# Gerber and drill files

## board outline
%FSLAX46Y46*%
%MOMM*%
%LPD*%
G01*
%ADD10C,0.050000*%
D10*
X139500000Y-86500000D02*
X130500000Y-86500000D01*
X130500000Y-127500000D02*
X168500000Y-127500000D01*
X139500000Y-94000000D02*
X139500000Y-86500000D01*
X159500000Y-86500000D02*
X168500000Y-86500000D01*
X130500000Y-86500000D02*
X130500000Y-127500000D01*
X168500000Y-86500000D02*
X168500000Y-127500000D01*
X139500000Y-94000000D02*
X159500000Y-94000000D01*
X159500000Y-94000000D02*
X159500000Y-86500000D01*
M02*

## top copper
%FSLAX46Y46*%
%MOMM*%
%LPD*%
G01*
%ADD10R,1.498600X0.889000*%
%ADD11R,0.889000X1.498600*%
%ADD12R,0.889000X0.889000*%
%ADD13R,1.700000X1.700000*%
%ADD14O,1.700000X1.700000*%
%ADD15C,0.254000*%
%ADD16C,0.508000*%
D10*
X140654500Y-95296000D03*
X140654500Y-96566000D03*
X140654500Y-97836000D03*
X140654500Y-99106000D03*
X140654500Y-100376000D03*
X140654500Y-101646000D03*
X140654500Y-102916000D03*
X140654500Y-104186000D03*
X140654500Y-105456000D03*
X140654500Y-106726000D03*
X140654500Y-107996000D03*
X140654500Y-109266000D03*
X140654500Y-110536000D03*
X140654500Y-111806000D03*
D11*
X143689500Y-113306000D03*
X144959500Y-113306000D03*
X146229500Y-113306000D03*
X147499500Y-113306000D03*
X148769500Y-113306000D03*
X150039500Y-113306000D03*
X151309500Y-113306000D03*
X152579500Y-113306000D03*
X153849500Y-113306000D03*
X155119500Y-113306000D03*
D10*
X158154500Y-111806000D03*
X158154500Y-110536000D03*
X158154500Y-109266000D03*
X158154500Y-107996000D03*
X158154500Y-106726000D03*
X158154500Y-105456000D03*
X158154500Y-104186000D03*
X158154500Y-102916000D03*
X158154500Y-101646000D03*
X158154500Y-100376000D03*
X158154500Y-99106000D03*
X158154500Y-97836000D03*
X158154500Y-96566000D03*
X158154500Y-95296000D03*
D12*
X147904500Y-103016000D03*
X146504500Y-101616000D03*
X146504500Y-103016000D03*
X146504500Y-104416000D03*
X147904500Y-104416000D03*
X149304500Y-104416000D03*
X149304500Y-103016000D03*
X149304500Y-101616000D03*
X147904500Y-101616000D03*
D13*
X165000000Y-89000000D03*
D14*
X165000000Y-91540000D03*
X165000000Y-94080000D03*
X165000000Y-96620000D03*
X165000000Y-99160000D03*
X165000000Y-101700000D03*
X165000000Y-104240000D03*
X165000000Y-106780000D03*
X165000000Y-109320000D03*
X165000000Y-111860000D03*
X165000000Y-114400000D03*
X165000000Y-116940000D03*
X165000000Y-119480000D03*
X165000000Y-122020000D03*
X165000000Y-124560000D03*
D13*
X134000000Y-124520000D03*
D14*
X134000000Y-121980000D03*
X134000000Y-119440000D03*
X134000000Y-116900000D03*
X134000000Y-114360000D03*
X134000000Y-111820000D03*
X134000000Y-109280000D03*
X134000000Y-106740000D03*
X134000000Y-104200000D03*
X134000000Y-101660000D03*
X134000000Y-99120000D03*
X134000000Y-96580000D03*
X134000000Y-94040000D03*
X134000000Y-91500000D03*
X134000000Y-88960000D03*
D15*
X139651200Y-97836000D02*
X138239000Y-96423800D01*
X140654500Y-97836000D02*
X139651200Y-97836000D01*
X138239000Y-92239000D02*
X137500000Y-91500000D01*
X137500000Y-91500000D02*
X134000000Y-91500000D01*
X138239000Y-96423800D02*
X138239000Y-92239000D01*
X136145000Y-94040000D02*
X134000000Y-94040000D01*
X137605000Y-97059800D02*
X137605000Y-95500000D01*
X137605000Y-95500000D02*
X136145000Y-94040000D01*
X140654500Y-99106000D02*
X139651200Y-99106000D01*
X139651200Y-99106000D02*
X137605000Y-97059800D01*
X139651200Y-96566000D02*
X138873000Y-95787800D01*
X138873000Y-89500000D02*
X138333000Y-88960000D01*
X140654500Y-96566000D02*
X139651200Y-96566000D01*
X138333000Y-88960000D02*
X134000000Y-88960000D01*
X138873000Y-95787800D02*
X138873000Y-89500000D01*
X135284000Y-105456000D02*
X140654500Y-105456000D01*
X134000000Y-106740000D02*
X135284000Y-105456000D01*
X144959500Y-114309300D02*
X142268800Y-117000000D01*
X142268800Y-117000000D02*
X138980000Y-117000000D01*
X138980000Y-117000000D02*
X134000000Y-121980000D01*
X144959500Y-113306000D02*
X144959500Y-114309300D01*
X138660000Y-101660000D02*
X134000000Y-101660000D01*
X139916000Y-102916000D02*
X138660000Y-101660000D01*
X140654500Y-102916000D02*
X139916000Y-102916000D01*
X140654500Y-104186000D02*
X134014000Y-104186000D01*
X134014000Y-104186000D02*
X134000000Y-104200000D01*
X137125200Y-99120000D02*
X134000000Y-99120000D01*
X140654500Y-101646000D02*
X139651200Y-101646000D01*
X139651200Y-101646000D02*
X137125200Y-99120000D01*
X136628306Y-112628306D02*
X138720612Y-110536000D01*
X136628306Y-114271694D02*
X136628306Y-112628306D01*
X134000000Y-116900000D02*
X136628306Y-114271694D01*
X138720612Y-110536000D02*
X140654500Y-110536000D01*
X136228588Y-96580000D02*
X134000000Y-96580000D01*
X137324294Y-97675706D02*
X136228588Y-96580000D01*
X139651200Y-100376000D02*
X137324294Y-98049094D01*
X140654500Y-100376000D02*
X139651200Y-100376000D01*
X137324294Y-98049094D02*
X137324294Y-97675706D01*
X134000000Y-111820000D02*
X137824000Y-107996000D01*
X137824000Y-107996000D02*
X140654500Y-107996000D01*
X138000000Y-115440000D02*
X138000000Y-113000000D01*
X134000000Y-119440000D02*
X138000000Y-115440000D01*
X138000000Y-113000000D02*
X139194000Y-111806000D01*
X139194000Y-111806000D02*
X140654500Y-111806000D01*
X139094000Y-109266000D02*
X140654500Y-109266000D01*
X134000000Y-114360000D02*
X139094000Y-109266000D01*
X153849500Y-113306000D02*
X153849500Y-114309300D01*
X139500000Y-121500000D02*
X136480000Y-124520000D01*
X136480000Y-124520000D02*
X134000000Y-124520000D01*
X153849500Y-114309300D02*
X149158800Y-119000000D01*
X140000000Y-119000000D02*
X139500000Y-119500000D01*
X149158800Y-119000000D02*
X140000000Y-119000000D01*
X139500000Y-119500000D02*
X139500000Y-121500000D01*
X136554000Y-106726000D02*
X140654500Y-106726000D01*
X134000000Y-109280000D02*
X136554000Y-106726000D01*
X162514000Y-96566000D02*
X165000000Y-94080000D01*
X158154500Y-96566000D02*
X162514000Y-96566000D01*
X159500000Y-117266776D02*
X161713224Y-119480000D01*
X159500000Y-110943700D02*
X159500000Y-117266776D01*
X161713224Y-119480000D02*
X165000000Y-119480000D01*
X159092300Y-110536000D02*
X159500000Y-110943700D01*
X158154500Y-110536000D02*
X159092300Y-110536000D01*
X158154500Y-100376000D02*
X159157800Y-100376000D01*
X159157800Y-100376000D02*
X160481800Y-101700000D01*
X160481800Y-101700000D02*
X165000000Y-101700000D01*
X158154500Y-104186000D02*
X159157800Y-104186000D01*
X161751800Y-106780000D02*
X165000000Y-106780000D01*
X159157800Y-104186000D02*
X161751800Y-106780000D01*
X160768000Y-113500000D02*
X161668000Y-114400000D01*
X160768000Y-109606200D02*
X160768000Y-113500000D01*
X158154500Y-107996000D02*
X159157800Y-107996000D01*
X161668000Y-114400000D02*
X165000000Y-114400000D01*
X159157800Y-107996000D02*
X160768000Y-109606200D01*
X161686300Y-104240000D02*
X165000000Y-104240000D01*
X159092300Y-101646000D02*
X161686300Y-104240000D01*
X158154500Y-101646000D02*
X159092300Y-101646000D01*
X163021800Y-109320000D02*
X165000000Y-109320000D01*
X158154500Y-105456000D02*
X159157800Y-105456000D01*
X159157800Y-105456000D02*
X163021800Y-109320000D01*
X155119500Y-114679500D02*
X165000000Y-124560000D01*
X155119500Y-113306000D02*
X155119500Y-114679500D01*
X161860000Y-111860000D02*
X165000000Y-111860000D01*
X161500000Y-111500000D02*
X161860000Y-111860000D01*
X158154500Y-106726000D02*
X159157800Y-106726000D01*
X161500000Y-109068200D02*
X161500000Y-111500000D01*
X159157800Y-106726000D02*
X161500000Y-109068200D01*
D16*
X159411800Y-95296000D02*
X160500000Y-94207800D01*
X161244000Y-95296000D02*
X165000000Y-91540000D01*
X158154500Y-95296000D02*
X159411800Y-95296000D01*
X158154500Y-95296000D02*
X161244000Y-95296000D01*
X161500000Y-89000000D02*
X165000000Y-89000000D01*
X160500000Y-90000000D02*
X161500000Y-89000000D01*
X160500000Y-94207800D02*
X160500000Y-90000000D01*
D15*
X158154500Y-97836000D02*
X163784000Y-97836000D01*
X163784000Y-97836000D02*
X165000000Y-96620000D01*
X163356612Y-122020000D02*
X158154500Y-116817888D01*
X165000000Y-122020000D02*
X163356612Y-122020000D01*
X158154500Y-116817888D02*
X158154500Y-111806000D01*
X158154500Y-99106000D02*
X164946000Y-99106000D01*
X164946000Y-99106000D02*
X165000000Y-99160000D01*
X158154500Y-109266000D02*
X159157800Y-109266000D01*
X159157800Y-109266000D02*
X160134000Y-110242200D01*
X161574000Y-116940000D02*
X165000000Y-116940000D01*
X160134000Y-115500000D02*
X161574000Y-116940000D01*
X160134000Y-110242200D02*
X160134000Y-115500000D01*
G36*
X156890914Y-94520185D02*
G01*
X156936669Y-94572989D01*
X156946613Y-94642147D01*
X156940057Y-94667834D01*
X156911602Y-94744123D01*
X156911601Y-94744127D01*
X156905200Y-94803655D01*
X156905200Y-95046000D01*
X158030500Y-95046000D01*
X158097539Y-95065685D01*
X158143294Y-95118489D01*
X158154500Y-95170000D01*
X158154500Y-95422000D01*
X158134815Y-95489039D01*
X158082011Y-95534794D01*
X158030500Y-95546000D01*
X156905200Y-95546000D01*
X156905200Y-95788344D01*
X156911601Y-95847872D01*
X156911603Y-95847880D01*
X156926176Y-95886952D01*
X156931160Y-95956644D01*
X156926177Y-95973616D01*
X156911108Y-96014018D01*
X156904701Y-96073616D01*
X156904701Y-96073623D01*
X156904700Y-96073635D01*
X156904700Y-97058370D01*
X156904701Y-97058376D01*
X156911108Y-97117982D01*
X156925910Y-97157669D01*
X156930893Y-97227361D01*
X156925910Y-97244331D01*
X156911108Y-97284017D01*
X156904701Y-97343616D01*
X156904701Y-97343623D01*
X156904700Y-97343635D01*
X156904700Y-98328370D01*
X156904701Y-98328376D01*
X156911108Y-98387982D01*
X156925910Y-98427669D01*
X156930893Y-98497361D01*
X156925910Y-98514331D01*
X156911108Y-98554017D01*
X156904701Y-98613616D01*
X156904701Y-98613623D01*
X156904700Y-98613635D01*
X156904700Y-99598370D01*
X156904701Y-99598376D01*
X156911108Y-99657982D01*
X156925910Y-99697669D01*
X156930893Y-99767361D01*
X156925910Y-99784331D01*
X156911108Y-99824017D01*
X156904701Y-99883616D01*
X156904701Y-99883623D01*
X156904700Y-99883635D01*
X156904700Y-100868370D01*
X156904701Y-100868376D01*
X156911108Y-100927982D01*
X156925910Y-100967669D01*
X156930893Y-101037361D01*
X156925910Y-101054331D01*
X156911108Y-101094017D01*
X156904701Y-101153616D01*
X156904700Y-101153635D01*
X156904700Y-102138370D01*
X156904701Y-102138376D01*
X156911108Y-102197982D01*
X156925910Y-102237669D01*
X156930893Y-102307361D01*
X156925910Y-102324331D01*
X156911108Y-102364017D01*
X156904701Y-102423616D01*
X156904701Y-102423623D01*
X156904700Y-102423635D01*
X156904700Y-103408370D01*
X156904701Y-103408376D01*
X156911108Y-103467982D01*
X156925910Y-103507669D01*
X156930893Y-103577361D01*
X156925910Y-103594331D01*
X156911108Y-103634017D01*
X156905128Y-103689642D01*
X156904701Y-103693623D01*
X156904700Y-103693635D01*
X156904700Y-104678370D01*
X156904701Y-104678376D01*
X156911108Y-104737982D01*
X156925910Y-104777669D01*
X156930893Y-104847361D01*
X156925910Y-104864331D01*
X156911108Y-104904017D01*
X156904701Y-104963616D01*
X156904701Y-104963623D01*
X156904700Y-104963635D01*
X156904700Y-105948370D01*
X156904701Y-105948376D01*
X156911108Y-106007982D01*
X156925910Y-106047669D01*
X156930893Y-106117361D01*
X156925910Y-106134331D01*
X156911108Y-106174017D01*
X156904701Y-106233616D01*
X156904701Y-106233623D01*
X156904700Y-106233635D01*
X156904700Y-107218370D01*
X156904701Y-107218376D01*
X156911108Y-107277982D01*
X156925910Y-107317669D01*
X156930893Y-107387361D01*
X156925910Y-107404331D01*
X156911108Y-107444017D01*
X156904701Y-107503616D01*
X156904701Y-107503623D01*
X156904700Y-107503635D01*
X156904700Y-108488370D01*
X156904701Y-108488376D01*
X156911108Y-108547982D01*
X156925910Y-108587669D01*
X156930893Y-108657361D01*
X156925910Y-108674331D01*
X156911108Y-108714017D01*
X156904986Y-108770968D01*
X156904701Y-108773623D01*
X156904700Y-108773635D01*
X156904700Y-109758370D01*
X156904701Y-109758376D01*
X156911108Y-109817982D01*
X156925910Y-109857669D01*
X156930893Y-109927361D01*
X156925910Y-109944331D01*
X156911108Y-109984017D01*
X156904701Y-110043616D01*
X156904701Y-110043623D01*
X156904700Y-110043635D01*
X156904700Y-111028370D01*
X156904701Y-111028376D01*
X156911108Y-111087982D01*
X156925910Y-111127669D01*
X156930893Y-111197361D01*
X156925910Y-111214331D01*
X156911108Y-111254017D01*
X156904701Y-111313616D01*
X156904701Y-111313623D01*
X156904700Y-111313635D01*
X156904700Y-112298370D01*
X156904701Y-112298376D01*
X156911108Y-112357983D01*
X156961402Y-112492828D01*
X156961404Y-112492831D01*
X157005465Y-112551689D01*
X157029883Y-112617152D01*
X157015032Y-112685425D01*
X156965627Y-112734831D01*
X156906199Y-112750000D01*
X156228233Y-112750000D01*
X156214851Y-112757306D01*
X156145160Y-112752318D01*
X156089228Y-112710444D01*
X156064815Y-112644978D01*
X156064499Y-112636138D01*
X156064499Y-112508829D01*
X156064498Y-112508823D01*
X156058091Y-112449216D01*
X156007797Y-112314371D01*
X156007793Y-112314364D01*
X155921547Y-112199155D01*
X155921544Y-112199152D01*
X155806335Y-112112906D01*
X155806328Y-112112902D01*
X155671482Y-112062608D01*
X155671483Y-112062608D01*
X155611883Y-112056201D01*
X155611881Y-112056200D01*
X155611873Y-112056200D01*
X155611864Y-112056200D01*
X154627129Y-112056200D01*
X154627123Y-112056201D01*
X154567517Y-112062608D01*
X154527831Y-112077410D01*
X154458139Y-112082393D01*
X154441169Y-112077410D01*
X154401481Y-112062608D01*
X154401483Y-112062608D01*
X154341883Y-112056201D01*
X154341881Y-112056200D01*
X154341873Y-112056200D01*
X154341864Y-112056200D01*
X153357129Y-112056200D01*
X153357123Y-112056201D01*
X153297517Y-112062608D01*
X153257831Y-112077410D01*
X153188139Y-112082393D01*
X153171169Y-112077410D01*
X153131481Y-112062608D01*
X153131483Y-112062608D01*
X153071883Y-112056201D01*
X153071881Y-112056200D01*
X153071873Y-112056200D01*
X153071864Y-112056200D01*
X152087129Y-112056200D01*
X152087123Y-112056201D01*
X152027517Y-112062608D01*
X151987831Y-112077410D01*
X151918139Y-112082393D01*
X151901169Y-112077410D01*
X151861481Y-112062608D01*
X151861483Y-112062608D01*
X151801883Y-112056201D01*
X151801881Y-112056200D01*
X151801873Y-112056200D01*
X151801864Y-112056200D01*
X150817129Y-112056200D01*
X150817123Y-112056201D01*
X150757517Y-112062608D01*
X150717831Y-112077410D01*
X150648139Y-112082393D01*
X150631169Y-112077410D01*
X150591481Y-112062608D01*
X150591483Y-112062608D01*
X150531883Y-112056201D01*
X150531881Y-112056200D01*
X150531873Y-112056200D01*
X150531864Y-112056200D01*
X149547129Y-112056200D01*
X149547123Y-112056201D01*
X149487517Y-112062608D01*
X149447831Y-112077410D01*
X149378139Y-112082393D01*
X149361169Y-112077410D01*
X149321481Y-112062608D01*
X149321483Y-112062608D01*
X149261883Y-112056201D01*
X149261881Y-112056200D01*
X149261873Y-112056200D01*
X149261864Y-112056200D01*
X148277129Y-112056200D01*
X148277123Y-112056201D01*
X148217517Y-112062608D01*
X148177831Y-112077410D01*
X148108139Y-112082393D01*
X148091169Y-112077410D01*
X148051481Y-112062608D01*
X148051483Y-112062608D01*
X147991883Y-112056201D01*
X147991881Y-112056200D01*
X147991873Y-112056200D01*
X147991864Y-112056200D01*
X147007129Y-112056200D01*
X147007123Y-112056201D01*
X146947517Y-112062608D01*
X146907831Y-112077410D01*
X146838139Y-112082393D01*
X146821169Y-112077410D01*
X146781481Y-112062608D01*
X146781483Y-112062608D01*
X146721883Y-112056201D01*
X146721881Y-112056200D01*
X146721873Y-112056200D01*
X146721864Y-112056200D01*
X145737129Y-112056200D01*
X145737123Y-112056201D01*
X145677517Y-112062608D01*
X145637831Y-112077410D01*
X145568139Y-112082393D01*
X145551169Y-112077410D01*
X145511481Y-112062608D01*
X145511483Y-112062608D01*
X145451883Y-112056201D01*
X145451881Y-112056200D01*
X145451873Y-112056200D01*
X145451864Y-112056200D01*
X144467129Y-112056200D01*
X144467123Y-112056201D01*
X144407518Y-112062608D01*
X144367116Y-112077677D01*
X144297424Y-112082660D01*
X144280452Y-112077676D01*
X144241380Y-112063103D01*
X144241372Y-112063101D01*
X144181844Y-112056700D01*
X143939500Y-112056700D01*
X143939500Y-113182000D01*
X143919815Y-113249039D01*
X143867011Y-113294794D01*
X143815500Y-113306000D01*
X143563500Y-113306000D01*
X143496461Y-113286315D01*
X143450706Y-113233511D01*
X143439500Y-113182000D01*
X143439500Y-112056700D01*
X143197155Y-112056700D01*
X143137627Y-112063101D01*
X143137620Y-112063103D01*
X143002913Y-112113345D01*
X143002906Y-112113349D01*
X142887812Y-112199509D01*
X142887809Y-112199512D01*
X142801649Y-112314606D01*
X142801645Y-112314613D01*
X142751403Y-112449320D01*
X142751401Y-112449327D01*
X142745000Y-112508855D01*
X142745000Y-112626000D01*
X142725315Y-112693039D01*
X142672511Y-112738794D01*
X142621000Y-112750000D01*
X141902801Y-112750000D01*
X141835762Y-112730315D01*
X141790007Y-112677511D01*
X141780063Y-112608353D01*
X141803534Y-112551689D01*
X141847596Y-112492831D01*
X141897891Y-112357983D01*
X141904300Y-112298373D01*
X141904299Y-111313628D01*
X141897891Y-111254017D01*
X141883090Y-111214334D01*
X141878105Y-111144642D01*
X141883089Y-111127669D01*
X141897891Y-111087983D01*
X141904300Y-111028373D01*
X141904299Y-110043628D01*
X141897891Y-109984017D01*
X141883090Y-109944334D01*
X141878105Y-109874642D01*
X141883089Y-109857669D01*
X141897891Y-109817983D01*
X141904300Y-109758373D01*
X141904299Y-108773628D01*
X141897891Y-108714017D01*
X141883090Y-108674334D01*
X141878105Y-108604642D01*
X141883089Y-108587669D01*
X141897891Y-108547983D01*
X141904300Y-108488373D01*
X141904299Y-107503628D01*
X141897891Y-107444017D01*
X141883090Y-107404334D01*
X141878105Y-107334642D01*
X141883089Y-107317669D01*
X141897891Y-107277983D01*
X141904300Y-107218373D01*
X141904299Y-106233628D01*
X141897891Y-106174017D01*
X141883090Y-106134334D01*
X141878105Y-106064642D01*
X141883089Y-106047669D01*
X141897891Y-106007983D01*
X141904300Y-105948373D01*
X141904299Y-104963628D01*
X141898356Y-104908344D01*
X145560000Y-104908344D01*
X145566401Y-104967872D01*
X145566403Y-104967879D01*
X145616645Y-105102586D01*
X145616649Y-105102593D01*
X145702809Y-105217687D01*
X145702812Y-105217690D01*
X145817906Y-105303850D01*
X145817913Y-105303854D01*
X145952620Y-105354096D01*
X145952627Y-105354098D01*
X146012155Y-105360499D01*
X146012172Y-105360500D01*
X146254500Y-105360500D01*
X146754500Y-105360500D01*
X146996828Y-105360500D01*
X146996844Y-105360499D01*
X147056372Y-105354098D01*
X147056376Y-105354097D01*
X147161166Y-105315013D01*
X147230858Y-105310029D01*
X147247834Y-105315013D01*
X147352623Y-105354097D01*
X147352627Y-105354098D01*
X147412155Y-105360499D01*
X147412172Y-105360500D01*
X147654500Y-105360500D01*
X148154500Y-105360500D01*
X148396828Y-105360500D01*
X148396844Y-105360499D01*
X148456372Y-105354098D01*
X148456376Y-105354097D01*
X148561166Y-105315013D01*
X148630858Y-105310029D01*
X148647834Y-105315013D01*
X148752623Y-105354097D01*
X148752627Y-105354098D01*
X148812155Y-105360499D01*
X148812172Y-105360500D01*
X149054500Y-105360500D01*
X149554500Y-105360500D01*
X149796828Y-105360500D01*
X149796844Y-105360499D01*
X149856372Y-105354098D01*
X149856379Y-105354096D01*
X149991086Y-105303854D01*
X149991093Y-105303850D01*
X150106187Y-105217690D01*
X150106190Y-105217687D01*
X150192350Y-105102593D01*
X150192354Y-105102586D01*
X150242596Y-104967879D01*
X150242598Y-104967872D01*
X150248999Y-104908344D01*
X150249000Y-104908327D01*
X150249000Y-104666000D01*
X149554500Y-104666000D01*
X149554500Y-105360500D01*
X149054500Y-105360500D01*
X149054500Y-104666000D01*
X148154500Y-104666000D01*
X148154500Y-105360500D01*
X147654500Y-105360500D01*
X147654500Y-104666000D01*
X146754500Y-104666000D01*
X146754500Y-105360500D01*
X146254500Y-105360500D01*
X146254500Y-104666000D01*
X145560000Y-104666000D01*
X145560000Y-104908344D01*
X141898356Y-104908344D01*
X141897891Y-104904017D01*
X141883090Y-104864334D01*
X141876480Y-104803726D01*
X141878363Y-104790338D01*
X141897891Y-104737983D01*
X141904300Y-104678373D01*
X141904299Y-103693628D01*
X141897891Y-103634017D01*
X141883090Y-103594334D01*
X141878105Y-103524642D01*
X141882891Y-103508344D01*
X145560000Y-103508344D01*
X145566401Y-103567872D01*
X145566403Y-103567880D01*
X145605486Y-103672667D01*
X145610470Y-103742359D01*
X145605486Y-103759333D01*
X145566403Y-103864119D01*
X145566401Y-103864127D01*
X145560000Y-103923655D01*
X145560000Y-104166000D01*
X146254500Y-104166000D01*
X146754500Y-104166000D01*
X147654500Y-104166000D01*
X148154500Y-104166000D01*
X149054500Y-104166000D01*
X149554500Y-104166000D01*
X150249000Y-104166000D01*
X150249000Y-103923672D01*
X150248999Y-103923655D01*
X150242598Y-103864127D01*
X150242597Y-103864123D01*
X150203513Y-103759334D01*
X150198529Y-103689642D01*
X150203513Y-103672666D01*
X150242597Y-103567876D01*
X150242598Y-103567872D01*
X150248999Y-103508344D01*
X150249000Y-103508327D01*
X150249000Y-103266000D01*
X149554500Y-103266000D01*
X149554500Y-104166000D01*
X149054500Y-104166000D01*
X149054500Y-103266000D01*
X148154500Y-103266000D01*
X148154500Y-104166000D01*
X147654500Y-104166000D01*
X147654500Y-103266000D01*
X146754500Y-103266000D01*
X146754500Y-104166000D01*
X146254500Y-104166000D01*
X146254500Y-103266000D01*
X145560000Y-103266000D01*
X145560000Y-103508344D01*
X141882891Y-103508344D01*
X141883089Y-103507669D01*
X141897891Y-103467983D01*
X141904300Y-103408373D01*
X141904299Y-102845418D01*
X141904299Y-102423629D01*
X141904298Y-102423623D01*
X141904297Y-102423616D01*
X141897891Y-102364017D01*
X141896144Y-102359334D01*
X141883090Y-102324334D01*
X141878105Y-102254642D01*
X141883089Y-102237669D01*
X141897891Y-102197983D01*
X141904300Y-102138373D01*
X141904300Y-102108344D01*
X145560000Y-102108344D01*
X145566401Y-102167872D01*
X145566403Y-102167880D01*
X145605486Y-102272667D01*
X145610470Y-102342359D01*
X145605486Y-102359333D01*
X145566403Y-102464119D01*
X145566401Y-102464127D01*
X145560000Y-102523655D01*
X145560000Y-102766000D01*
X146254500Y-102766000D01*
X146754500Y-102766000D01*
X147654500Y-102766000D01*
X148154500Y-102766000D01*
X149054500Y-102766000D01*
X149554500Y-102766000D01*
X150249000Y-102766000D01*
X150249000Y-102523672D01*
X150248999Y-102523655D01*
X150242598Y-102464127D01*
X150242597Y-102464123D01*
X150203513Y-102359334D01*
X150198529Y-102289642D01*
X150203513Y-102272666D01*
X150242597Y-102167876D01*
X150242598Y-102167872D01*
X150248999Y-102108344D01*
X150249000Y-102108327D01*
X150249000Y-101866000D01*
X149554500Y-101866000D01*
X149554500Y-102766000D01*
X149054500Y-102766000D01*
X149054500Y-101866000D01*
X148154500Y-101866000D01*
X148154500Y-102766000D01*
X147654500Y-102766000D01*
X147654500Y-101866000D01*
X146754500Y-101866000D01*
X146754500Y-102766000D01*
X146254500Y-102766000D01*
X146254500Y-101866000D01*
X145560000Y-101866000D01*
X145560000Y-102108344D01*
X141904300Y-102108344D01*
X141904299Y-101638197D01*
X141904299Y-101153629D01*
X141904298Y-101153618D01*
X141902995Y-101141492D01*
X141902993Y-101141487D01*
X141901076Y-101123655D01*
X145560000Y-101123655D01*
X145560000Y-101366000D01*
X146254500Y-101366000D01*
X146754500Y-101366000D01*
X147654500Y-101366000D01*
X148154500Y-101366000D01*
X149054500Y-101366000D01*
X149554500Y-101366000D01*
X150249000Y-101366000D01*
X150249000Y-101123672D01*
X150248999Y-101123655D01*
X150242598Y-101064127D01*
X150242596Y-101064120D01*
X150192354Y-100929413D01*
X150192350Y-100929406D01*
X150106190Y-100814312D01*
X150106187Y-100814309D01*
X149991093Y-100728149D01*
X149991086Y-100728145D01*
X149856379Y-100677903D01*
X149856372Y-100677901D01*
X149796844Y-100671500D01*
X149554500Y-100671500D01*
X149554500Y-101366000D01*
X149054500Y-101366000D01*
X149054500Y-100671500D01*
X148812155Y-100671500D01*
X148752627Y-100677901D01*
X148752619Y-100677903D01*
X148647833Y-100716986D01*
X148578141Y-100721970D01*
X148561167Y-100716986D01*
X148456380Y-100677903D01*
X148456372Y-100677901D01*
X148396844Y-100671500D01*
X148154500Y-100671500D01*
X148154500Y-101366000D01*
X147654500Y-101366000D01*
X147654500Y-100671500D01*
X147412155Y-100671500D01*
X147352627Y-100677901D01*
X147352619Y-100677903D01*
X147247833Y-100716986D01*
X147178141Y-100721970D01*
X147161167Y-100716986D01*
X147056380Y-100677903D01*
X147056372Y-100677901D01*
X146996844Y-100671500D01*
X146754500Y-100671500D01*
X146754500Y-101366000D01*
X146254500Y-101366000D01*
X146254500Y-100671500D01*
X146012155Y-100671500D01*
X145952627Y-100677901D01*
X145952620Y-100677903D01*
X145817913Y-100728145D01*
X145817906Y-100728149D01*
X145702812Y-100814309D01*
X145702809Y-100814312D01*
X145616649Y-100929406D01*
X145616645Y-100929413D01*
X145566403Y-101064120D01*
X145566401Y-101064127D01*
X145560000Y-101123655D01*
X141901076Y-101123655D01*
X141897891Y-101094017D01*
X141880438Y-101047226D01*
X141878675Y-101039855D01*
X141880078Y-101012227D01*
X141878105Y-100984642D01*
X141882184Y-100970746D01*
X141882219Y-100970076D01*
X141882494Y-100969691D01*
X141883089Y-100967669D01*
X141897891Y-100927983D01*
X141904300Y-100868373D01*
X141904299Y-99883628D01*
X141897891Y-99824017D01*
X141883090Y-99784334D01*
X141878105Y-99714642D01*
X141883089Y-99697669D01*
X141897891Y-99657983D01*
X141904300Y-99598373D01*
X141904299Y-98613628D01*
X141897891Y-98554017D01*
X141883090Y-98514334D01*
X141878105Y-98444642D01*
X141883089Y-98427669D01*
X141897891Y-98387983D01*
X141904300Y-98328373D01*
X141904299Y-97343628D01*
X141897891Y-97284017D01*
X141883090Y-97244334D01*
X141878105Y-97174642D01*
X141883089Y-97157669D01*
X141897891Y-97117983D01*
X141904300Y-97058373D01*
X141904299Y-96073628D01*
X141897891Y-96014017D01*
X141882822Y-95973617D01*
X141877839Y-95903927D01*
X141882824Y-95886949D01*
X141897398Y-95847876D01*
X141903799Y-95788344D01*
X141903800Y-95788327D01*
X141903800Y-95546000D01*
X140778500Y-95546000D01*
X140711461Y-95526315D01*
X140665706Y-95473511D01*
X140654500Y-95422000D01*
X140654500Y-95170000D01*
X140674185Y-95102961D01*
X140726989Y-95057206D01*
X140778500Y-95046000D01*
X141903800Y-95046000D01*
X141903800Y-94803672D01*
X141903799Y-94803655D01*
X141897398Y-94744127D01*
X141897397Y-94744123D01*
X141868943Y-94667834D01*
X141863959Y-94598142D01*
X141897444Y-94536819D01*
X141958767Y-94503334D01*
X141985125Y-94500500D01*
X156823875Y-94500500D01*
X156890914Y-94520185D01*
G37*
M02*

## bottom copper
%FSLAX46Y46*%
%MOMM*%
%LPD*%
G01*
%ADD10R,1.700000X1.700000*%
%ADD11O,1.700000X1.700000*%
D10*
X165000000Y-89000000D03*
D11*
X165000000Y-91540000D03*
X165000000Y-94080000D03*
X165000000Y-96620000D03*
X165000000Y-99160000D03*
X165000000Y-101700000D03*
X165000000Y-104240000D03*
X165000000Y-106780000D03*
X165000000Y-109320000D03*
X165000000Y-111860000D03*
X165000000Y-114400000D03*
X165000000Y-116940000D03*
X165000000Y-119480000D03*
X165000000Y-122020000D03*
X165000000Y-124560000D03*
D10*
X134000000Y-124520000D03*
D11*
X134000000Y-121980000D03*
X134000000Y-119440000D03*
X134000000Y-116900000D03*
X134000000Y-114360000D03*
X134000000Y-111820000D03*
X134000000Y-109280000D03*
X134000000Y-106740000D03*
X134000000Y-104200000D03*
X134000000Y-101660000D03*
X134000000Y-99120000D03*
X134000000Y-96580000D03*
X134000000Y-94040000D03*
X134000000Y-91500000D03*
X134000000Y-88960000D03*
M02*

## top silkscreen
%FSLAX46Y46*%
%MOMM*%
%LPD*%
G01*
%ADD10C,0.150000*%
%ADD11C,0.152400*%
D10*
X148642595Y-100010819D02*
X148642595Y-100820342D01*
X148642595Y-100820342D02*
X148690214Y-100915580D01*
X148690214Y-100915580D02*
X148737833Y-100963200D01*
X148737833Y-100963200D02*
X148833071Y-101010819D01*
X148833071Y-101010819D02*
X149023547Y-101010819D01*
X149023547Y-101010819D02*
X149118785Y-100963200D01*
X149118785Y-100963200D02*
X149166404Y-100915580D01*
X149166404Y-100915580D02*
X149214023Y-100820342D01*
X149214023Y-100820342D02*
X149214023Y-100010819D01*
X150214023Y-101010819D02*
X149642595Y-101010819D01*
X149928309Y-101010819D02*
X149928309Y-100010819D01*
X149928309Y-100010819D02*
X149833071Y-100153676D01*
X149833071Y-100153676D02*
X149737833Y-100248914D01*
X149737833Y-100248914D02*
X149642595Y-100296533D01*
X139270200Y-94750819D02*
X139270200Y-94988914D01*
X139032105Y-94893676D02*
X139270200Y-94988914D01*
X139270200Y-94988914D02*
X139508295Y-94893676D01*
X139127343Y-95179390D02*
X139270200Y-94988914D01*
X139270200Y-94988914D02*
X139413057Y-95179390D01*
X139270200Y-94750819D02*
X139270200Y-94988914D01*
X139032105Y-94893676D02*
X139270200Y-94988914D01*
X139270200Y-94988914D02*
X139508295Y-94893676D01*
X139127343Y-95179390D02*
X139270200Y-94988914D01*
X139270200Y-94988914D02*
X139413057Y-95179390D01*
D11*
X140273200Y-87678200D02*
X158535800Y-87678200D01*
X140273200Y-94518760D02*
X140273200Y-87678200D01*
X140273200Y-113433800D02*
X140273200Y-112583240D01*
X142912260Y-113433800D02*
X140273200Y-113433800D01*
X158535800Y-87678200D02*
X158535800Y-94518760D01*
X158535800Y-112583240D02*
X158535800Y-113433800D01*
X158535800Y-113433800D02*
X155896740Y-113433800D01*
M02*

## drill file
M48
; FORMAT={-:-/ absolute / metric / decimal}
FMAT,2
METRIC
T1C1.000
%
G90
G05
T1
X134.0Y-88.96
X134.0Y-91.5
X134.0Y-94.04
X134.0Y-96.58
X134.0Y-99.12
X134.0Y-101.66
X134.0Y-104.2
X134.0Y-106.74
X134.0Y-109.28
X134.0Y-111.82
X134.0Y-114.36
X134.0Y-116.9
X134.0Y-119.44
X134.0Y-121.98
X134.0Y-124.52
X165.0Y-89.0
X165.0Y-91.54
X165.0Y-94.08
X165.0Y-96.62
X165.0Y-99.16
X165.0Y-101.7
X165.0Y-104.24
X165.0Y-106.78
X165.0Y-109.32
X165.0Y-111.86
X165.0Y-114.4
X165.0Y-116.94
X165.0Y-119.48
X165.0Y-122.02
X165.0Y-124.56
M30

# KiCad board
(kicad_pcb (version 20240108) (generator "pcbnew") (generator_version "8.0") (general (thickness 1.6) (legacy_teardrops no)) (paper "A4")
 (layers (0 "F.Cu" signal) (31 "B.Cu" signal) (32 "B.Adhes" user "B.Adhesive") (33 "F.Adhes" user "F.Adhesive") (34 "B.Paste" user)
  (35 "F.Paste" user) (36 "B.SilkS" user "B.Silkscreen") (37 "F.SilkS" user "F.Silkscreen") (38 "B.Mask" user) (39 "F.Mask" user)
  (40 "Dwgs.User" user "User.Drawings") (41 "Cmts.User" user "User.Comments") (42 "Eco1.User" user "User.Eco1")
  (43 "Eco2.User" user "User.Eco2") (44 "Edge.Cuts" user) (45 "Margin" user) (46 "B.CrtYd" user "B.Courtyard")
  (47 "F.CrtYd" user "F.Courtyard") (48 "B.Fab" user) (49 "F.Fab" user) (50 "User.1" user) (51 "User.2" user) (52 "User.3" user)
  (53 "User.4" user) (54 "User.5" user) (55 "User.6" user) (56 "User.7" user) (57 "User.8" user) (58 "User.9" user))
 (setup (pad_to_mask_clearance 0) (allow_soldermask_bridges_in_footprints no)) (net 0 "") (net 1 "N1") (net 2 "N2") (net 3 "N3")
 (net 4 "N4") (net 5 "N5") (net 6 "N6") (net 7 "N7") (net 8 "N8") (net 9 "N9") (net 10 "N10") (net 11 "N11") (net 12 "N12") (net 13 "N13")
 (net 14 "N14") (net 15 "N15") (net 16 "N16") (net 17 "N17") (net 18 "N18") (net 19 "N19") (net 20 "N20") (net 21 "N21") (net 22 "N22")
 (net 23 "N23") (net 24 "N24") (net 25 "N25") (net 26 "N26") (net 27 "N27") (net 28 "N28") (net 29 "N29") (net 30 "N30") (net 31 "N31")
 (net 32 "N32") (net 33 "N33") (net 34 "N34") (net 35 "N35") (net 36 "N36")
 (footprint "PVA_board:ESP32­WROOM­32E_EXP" (layer "F.Cu") (at 149.4045 100.556)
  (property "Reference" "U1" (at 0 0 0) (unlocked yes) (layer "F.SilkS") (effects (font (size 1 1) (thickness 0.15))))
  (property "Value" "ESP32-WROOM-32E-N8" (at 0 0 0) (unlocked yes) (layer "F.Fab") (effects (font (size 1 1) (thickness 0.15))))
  (fp_line (start -9.1313 -12.8778) (end 9.1313 -12.8778) (stroke (width 0.1524) (type solid)) (layer "F.SilkS"))
  (fp_line (start -9.1313 -6.03724) (end -9.1313 -12.8778) (stroke (width 0.1524) (type solid)) (layer "F.SilkS"))
  (fp_line (start -9.1313 12.8778) (end -9.1313 12.02724) (stroke (width 0.1524) (type solid)) (layer "F.SilkS"))
  (fp_line (start -6.49224 12.8778) (end -9.1313 12.8778) (stroke (width 0.1524) (type solid)) (layer "F.SilkS"))
  (fp_line (start 9.1313 -12.8778) (end 9.1313 -6.03724) (stroke (width 0.1524) (type solid)) (layer "F.SilkS"))
  (fp_line (start 9.1313 12.02724) (end 9.1313 12.8778) (stroke (width 0.1524) (type solid)) (layer "F.SilkS"))
  (fp_line (start 9.1313 12.8778) (end 6.49224 12.8778) (stroke (width 0.1524) (type solid)) (layer "F.SilkS"))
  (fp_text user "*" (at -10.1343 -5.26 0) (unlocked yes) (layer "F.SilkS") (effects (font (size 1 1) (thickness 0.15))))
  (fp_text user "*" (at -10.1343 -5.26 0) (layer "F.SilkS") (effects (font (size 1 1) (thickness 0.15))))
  (pad "1" smd rect (at -8.75 -5.26) (size 1.4986 0.889) (layers "F.Cu" "F.Paste" "F.Mask") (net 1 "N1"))
  (pad "2" smd rect (at -8.75 -3.99) (size 1.4986 0.889) (layers "F.Cu" "F.Paste" "F.Mask") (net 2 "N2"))
  (pad "3" smd rect (at -8.75 -2.72) (size 1.4986 0.889) (layers "F.Cu" "F.Paste" "F.Mask") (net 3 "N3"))
  (pad "4" smd rect (at -8.75 -1.45) (size 1.4986 0.889) (layers "F.Cu" "F.Paste" "F.Mask") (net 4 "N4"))
  (pad "5" smd rect (at -8.75 -0.18) (size 1.4986 0.889) (layers "F.Cu" "F.Paste" "F.Mask") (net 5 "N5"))
  (pad "6" smd rect (at -8.75 1.09) (size 1.4986 0.889) (layers "F.Cu" "F.Paste" "F.Mask") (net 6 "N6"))
  (pad "7" smd rect (at -8.75 2.36) (size 1.4986 0.889) (layers "F.Cu" "F.Paste" "F.Mask") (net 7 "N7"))
  (pad "8" smd rect (at -8.75 3.63) (size 1.4986 0.889) (layers "F.Cu" "F.Paste" "F.Mask") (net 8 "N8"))
  (pad "9" smd rect (at -8.75 4.9) (size 1.4986 0.889) (layers "F.Cu" "F.Paste" "F.Mask") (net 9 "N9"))
  (pad "10" smd rect (at -8.75 6.17) (size 1.4986 0.889) (layers "F.Cu" "F.Paste" "F.Mask") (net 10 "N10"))
  (pad "11" smd rect (at -8.75 7.44) (size 1.4986 0.889) (layers "F.Cu" "F.Paste" "F.Mask") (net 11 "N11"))
  (pad "12" smd rect (at -8.75 8.71) (size 1.4986 0.889) (layers "F.Cu" "F.Paste" "F.Mask") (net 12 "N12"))
  (pad "13" smd rect (at -8.75 9.98) (size 1.4986 0.889) (layers "F.Cu" "F.Paste" "F.Mask") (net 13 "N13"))
  (pad "14" smd rect (at -8.75 11.25) (size 1.4986 0.889) (layers "F.Cu" "F.Paste" "F.Mask") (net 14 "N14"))
  (pad "15" smd rect (at -5.715 12.75 90) (size 1.4986 0.889) (layers "F.Cu" "F.Paste" "F.Mask") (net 1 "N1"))
  (pad "16" smd rect (at -4.445 12.75 90) (size 1.4986 0.889) (layers "F.Cu" "F.Paste" "F.Mask") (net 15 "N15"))
  (pad "17" smd rect (at -3.175 12.75 90) (size 1.4986 0.889) (layers "F.Cu" "F.Paste" "F.Mask") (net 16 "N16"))
  (pad "18" smd rect (at -1.905 12.75 90) (size 1.4986 0.889) (layers "F.Cu" "F.Paste" "F.Mask") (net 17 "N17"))
  (pad "19" smd rect (at -0.635 12.75 90) (size 1.4986 0.889) (layers "F.Cu" "F.Paste" "F.Mask") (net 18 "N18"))
  (pad "20" smd rect (at 0.635 12.75 90) (size 1.4986 0.889) (layers "F.Cu" "F.Paste" "F.Mask") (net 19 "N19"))
  (pad "21" smd rect (at 1.905 12.75 90) (size 1.4986 0.889) (layers "F.Cu" "F.Paste" "F.Mask") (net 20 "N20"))
  (pad "22" smd rect (at 3.175 12.75 90) (size 1.4986 0.889) (layers "F.Cu" "F.Paste" "F.Mask") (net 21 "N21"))
  (pad "23" smd rect (at 4.445 12.75 90) (size 1.4986 0.889) (layers "F.Cu" "F.Paste" "F.Mask") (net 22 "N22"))
  (pad "24" smd rect (at 5.715 12.75 90) (size 1.4986 0.889) (layers "F.Cu" "F.Paste" "F.Mask") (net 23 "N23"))
  (pad "25" smd rect (at 8.75 11.25) (size 1.4986 0.889) (layers "F.Cu" "F.Paste" "F.Mask") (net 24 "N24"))
  (pad "26" smd rect (at 8.75 9.98) (size 1.4986 0.889) (layers "F.Cu" "F.Paste" "F.Mask") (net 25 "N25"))
  (pad "27" smd rect (at 8.75 8.71) (size 1.4986 0.889) (layers "F.Cu" "F.Paste" "F.Mask") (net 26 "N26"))
  (pad "28" smd rect (at 8.75 7.44) (size 1.4986 0.889) (layers "F.Cu" "F.Paste" "F.Mask") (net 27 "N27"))
  (pad "29" smd rect (at 8.75 6.17) (size 1.4986 0.889) (layers "F.Cu" "F.Paste" "F.Mask") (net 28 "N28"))
  (pad "30" smd rect (at 8.75 4.9) (size 1.4986 0.889) (layers "F.Cu" "F.Paste" "F.Mask") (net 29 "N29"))
  (pad "31" smd rect (at 8.75 3.63) (size 1.4986 0.889) (layers "F.Cu" "F.Paste" "F.Mask") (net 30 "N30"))
  (pad "32" smd rect (at 8.75 2.36) (size 1.4986 0.889) (layers "F.Cu" "F.Paste" "F.Mask") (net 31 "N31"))
  (pad "33" smd rect (at 8.75 1.09) (size 1.4986 0.889) (layers "F.Cu" "F.Paste" "F.Mask") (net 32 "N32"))
  (pad "34" smd rect (at 8.75 -0.18) (size 1.4986 0.889) (layers "F.Cu" "F.Paste" "F.Mask") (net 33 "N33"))
  (pad "35" smd rect (at 8.75 -1.45) (size 1.4986 0.889) (layers "F.Cu" "F.Paste" "F.Mask") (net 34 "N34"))
  (pad "36" smd rect (at 8.75 -2.72) (size 1.4986 0.889) (layers "F.Cu" "F.Paste" "F.Mask") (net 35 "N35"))
  (pad "37" smd rect (at 8.75 -3.99) (size 1.4986 0.889) (layers "F.Cu" "F.Paste" "F.Mask") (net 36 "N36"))
  (pad "38" smd rect (at 8.75 -5.26) (size 1.4986 0.889) (layers "F.Cu" "F.Paste" "F.Mask") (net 1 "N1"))
  (pad "39" smd rect (at -1.5 2.46) (size 0.889 0.889) (layers "F.Cu" "F.Paste" "F.Mask") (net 1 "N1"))
  (pad "40" smd rect (at -2.9 1.06) (size 0.889 0.889) (layers "F.Cu" "F.Paste" "F.Mask") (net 1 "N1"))
  (pad "41" smd rect (at -2.9 2.46) (size 0.889 0.889) (layers "F.Cu" "F.Paste" "F.Mask") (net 1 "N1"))
  (pad "42" smd rect (at -2.9 3.86) (size 0.889 0.889) (layers "F.Cu" "F.Paste" "F.Mask") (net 1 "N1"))
  (pad "43" smd rect (at -1.5 3.86) (size 0.889 0.889) (layers "F.Cu" "F.Paste" "F.Mask") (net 1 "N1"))
  (pad "44" smd rect (at -0.1 3.86) (size 0.889 0.889) (layers "F.Cu" "F.Paste" "F.Mask") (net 1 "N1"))
  (pad "45" smd rect (at -0.1 2.46) (size 0.889 0.889) (layers "F.Cu" "F.Paste" "F.Mask") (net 1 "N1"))
  (pad "46" smd rect (at -0.1 1.06) (size 0.889 0.889) (layers "F.Cu" "F.Paste" "F.Mask") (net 1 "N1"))
  (pad "47" smd rect (at -1.5 1.06) (size 0.889 0.889) (layers "F.Cu" "F.Paste" "F.Mask") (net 1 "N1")))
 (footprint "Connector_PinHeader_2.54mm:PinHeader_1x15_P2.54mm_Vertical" (layer "B.Cu") (at 165 89 180)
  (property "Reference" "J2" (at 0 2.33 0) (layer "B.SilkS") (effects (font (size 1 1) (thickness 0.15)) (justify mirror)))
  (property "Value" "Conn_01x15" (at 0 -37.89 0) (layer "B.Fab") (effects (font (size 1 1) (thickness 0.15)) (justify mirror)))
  (pad "1" thru_hole rect (at 0 0 180) (size 1.7 1.7) (drill 1) (layers "*.Cu" "*.Mask") (remove_unused_layers no) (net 1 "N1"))
  (pad "2" thru_hole oval (at 0 -2.54 180) (size 1.7 1.7) (drill 1) (layers "*.Cu" "*.Mask") (remove_unused_layers no) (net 1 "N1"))
  (pad "3" thru_hole oval (at 0 -5.08 180) (size 1.7 1.7) (drill 1) (layers "*.Cu" "*.Mask") (remove_unused_layers no) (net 36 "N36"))
  (pad "4" thru_hole oval (at 0 -7.62 180) (size 1.7 1.7) (drill 1) (layers "*.Cu" "*.Mask") (remove_unused_layers no) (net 35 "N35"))
  (pad "5" thru_hole oval (at 0 -10.16 180) (size 1.7 1.7) (drill 1) (layers "*.Cu" "*.Mask") (remove_unused_layers no) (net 34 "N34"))
  (pad "6" thru_hole oval (at 0 -12.7 180) (size 1.7 1.7) (drill 1) (layers "*.Cu" "*.Mask") (remove_unused_layers no) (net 33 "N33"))
  (pad "7" thru_hole oval (at 0 -15.24 180) (size 1.7 1.7) (drill 1) (layers "*.Cu" "*.Mask") (remove_unused_layers no) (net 32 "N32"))
  (pad "8" thru_hole oval (at 0 -17.78 180) (size 1.7 1.7) (drill 1) (layers "*.Cu" "*.Mask") (remove_unused_layers no) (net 30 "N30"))
  (pad "9" thru_hole oval (at 0 -20.32 180) (size 1.7 1.7) (drill 1) (layers "*.Cu" "*.Mask") (remove_unused_layers no) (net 29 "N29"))
  (pad "10" thru_hole oval (at 0 -22.86 180) (size 1.7 1.7) (drill 1) (layers "*.Cu" "*.Mask") (remove_unused_layers no) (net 28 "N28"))
  (pad "11" thru_hole oval (at 0 -25.4 180) (size 1.7 1.7) (drill 1) (layers "*.Cu" "*.Mask") (remove_unused_layers no) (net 27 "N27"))
  (pad "12" thru_hole oval (at 0 -27.94 180) (size 1.7 1.7) (drill 1) (layers "*.Cu" "*.Mask") (remove_unused_layers no) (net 26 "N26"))
  (pad "13" thru_hole oval (at 0 -30.48 180) (size 1.7 1.7) (drill 1) (layers "*.Cu" "*.Mask") (remove_unused_layers no) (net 25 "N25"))
  (pad "14" thru_hole oval (at 0 -33.02 180) (size 1.7 1.7) (drill 1) (layers "*.Cu" "*.Mask") (remove_unused_layers no) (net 24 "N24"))
  (pad "15" thru_hole oval (at 0 -35.56 180) (size 1.7 1.7) (drill 1) (layers "*.Cu" "*.Mask") (remove_unused_layers no) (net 23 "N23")))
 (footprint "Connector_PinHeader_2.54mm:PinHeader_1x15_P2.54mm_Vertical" (layer "B.Cu") (at 134 124.52)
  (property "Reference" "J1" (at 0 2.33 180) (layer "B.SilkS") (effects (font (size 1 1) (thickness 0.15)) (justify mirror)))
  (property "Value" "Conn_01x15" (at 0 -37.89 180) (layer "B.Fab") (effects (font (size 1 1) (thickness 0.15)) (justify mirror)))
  (pad "1" thru_hole rect (at 0 0) (size 1.7 1.7) (drill 1) (layers "*.Cu" "*.Mask") (remove_unused_layers no) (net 22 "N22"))
  (pad "2" thru_hole oval (at 0 -2.54) (size 1.7 1.7) (drill 1) (layers "*.Cu" "*.Mask") (remove_unused_layers no) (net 15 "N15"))
  (pad "3" thru_hole oval (at 0 -5.08) (size 1.7 1.7) (drill 1) (layers "*.Cu" "*.Mask") (remove_unused_layers no) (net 14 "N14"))
  (pad "4" thru_hole oval (at 0 -7.62) (size 1.7 1.7) (drill 1) (layers "*.Cu" "*.Mask") (remove_unused_layers no) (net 13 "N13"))
  (pad "5" thru_hole oval (at 0 -10.16) (size 1.7 1.7) (drill 1) (layers "*.Cu" "*.Mask") (remove_unused_layers no) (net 12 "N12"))
  (pad "6" thru_hole oval (at 0 -12.7) (size 1.7 1.7) (drill 1) (layers "*.Cu" "*.Mask") (remove_unused_layers no) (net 11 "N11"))
  (pad "7" thru_hole oval (at 0 -15.24) (size 1.7 1.7) (drill 1) (layers "*.Cu" "*.Mask") (remove_unused_layers no) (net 10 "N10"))
  (pad "8" thru_hole oval (at 0 -17.78) (size 1.7 1.7) (drill 1) (layers "*.Cu" "*.Mask") (remove_unused_layers no) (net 9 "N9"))
  (pad "9" thru_hole oval (at 0 -20.32) (size 1.7 1.7) (drill 1) (layers "*.Cu" "*.Mask") (remove_unused_layers no) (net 8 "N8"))
  (pad "10" thru_hole oval (at 0 -22.86) (size 1.7 1.7) (drill 1) (layers "*.Cu" "*.Mask") (remove_unused_layers no) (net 7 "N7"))
  (pad "11" thru_hole oval (at 0 -25.4) (size 1.7 1.7) (drill 1) (layers "*.Cu" "*.Mask") (remove_unused_layers no) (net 6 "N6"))
  (pad "12" thru_hole oval (at 0 -27.94) (size 1.7 1.7) (drill 1) (layers "*.Cu" "*.Mask") (remove_unused_layers no) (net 5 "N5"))
  (pad "13" thru_hole oval (at 0 -30.48) (size 1.7 1.7) (drill 1) (layers "*.Cu" "*.Mask") (remove_unused_layers no) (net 4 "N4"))
  (pad "14" thru_hole oval (at 0 -33.02) (size 1.7 1.7) (drill 1) (layers "*.Cu" "*.Mask") (remove_unused_layers no) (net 3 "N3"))
  (pad "15" thru_hole oval (at 0 -35.56) (size 1.7 1.7) (drill 1) (layers "*.Cu" "*.Mask") (remove_unused_layers no) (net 2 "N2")))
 (gr_line (start 139.5 86.5) (end 130.5 86.5) (stroke (width 0.05) (type default)) (layer "Edge.Cuts"))
 (gr_line (start 130.5 127.5) (end 168.5 127.5) (stroke (width 0.05) (type default)) (layer "Edge.Cuts"))
 (gr_line (start 139.5 94) (end 139.5 86.5) (stroke (width 0.05) (type default)) (layer "Edge.Cuts"))
 (gr_line (start 159.5 86.5) (end 168.5 86.5) (stroke (width 0.05) (type default)) (layer "Edge.Cuts"))
 (gr_line (start 130.5 86.5) (end 130.5 127.5) (stroke (width 0.05) (type default)) (layer "Edge.Cuts"))
 (gr_line (start 168.5 86.5) (end 168.5 127.5) (stroke (width 0.05) (type default)) (layer "Edge.Cuts"))
 (gr_line (start 139.5 94) (end 159.5 94) (stroke (width 0.05) (type default)) (layer "Edge.Cuts"))
 (gr_line (start 159.5 94) (end 159.5 86.5) (stroke (width 0.05) (type default)) (layer "Edge.Cuts"))
 (segment (start 139.6512 97.836) (end 138.239 96.4238) (width 0.254) (layer "F.Cu") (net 3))
 (segment (start 140.6545 97.836) (end 139.6512 97.836) (width 0.254) (layer "F.Cu") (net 3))
 (segment (start 138.239 92.239) (end 137.5 91.5) (width 0.254) (layer "F.Cu") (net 3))
 (segment (start 137.5 91.5) (end 134 91.5) (width 0.254) (layer "F.Cu") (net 3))
 (segment (start 138.239 96.4238) (end 138.239 92.239) (width 0.254) (layer "F.Cu") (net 3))
 (segment (start 136.145 94.04) (end 134 94.04) (width 0.254) (layer "F.Cu") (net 4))
 (segment (start 137.605 97.0598) (end 137.605 95.5) (width 0.254) (layer "F.Cu") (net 4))
 (segment (start 137.605 95.5) (end 136.145 94.04) (width 0.254) (layer "F.Cu") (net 4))
 (segment (start 140.6545 99.106) (end 139.6512 99.106) (width 0.254) (layer "F.Cu") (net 4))
 (segment (start 139.6512 99.106) (end 137.605 97.0598) (width 0.254) (layer "F.Cu") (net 4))
 (segment (start 139.6512 96.566) (end 138.873 95.7878) (width 0.254) (layer "F.Cu") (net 2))
 (segment (start 138.873 89.5) (end 138.333 88.96) (width 0.254) (layer "F.Cu") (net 2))
 (segment (start 140.6545 96.566) (end 139.6512 96.566) (width 0.254) (layer "F.Cu") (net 2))
 (segment (start 138.333 88.96) (end 134 88.96) (width 0.254) (layer "F.Cu") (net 2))
 (segment (start 138.873 95.7878) (end 138.873 89.5) (width 0.254) (layer "F.Cu") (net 2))
 (segment (start 135.284 105.456) (end 140.6545 105.456) (width 0.254) (layer "F.Cu") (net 9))
 (segment (start 134 106.74) (end 135.284 105.456) (width 0.254) (layer "F.Cu") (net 9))
 (segment (start 144.9595 114.3093) (end 142.2688 117) (width 0.254) (layer "F.Cu") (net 15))
 (segment (start 142.2688 117) (end 138.98 117) (width 0.254) (layer "F.Cu") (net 15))
 (segment (start 138.98 117) (end 134 121.98) (width 0.254) (layer "F.Cu") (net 15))
 (segment (start 144.9595 113.306) (end 144.9595 114.3093) (width 0.254) (layer "F.Cu") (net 15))
 (segment (start 138.66 101.66) (end 134 101.66) (width 0.254) (layer "F.Cu") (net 7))
 (segment (start 139.916 102.916) (end 138.66 101.66) (width 0.254) (layer "F.Cu") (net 7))
 (segment (start 140.6545 102.916) (end 139.916 102.916) (width 0.254) (layer "F.Cu") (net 7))
 (segment (start 140.6545 104.186) (end 134.014 104.186) (width 0.254) (layer "F.Cu") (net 8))
 (segment (start 134.014 104.186) (end 134 104.2) (width 0.254) (layer "F.Cu") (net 8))
 (segment (start 137.1252 99.12) (end 134 99.12) (width 0.254) (layer "F.Cu") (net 6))
 (segment (start 140.6545 101.646) (end 139.6512 101.646) (width 0.254) (layer "F.Cu") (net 6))
 (segment (start 139.6512 101.646) (end 137.1252 99.12) (width 0.254) (layer "F.Cu") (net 6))
 (segment (start 136.628306 112.628306) (end 138.720612 110.536) (width 0.254) (layer "F.Cu") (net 13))
 (segment (start 136.628306 114.271694) (end 136.628306 112.628306) (width 0.254) (layer "F.Cu") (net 13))
 (segment (start 134 116.9) (end 136.628306 114.271694) (width 0.254) (layer "F.Cu") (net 13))
 (segment (start 138.720612 110.536) (end 140.6545 110.536) (width 0.254) (layer "F.Cu") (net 13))
 (segment (start 136.228588 96.58) (end 134 96.58) (width 0.254) (layer "F.Cu") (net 5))
 (segment (start 137.324294 97.675706) (end 136.228588 96.58) (width 0.254) (layer "F.Cu") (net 5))
 (segment (start 139.6512 100.376) (end 137.324294 98.049094) (width 0.254) (layer "F.Cu") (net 5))
 (segment (start 140.6545 100.376) (end 139.6512 100.376) (width 0.254) (layer "F.Cu") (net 5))
 (segment (start 137.324294 98.049094) (end 137.324294 97.675706) (width 0.254) (layer "F.Cu") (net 5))
 (segment (start 134 111.82) (end 137.824 107.996) (width 0.254) (layer "F.Cu") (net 11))
 (segment (start 137.824 107.996) (end 140.6545 107.996) (width 0.254) (layer "F.Cu") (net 11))
 (segment (start 138 115.44) (end 138 113) (width 0.254) (layer "F.Cu") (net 14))
 (segment (start 134 119.44) (end 138 115.44) (width 0.254) (layer "F.Cu") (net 14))
 (segment (start 138 113) (end 139.194 111.806) (width 0.254) (layer "F.Cu") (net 14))
 (segment (start 139.194 111.806) (end 140.6545 111.806) (width 0.254) (layer "F.Cu") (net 14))
 (segment (start 139.094 109.266) (end 140.6545 109.266) (width 0.254) (layer "F.Cu") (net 12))
 (segment (start 134 114.36) (end 139.094 109.266) (width 0.254) (layer "F.Cu") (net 12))
 (segment (start 153.8495 113.306) (end 153.8495 114.3093) (width 0.254) (layer "F.Cu") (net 22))
 (segment (start 139.5 121.5) (end 136.48 124.52) (width 0.254) (layer "F.Cu") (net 22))
 (segment (start 136.48 124.52) (end 134 124.52) (width 0.254) (layer "F.Cu") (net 22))
 (segment (start 153.8495 114.3093) (end 149.1588 119) (width 0.254) (layer "F.Cu") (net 22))
 (segment (start 140 119) (end 139.5 119.5) (width 0.254) (layer "F.Cu") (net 22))
 (segment (start 149.1588 119) (end 140 119) (width 0.254) (layer "F.Cu") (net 22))
 (segment (start 139.5 119.5) (end 139.5 121.5) (width 0.254) (layer "F.Cu") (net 22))
 (segment (start 136.554 106.726) (end 140.6545 106.726) (width 0.254) (layer "F.Cu") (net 10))
 (segment (start 134 109.28) (end 136.554 106.726) (width 0.254) (layer "F.Cu") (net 10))
 (segment (start 162.514 96.566) (end 165 94.08) (width 0.254) (layer "F.Cu") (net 36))
 (segment (start 158.1545 96.566) (end 162.514 96.566) (width 0.254) (layer "F.Cu") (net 36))
 (segment (start 159.5 117.266776) (end 161.713224 119.48) (width 0.254) (layer "F.Cu") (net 25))
 (segment (start 159.5 110.9437) (end 159.5 117.266776) (width 0.254) (layer "F.Cu") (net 25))
 (segment (start 161.713224 119.48) (end 165 119.48) (width 0.254) (layer "F.Cu") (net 25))
 (segment (start 159.0923 110.536) (end 159.5 110.9437) (width 0.254) (layer "F.Cu") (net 25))
 (segment (start 158.1545 110.536) (end 159.0923 110.536) (width 0.254) (layer "F.Cu") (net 25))
 (segment (start 158.1545 100.376) (end 159.1578 100.376) (width 0.254) (layer "F.Cu") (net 33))
 (segment (start 159.1578 100.376) (end 160.4818 101.7) (width 0.254) (layer "F.Cu") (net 33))
 (segment (start 160.4818 101.7) (end 165 101.7) (width 0.254) (layer "F.Cu") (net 33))
 (segment (start 158.1545 104.186) (end 159.1578 104.186) (width 0.254) (layer "F.Cu") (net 30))
 (segment (start 161.7518 106.78) (end 165 106.78) (width 0.254) (layer "F.Cu") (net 30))
 (segment (start 159.1578 104.186) (end 161.7518 106.78) (width 0.254) (layer "F.Cu") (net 30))
 (segment (start 160.768 113.5) (end 161.668 114.4) (width 0.254) (layer "F.Cu") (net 27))
 (segment (start 160.768 109.6062) (end 160.768 113.5) (width 0.254) (layer "F.Cu") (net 27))
 (segment (start 158.1545 107.996) (end 159.1578 107.996) (width 0.254) (layer "F.Cu") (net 27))
 (segment (start 161.668 114.4) (end 165 114.4) (width 0.254) (layer "F.Cu") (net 27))
 (segment (start 159.1578 107.996) (end 160.768 109.6062) (width 0.254) (layer "F.Cu") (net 27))
 (segment (start 161.6863 104.24) (end 165 104.24) (width 0.254) (layer "F.Cu") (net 32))
 (segment (start 159.0923 101.646) (end 161.6863 104.24) (width 0.254) (layer "F.Cu") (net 32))
 (segment (start 158.1545 101.646) (end 159.0923 101.646) (width 0.254) (layer "F.Cu") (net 32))
 (segment (start 163.0218 109.32) (end 165 109.32) (width 0.254) (layer "F.Cu") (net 29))
 (segment (start 158.1545 105.456) (end 159.1578 105.456) (width 0.254) (layer "F.Cu") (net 29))
 (segment (start 159.1578 105.456) (end 163.0218 109.32) (width 0.254) (layer "F.Cu") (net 29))
 (segment (start 155.1195 114.6795) (end 165 124.56) (width 0.254) (layer "F.Cu") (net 23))
 (segment (start 155.1195 113.306) (end 155.1195 114.6795) (width 0.254) (layer "F.Cu") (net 23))
 (segment (start 161.86 111.86) (end 165 111.86) (width 0.254) (layer "F.Cu") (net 28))
 (segment (start 161.5 111.5) (end 161.86 111.86) (width 0.254) (layer "F.Cu") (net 28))
 (segment (start 158.1545 106.726) (end 159.1578 106.726) (width 0.254) (layer "F.Cu") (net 28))
 (segment (start 161.5 109.0682) (end 161.5 111.5) (width 0.254) (layer "F.Cu") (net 28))
 (segment (start 159.1578 106.726) (end 161.5 109.0682) (width 0.254) (layer "F.Cu") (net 28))
 (segment (start 159.4118 95.296) (end 160.5 94.2078) (width 0.508) (layer "F.Cu") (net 1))
 (segment (start 161.244 95.296) (end 165 91.54) (width 0.508) (layer "F.Cu") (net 1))
 (segment (start 158.1545 95.296) (end 159.4118 95.296) (width 0.508) (layer "F.Cu") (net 1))
 (segment (start 158.1545 95.296) (end 161.244 95.296) (width 0.508) (layer "F.Cu") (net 1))
 (segment (start 161.5 89) (end 165 89) (width 0.508) (layer "F.Cu") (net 1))
 (segment (start 160.5 90) (end 161.5 89) (width 0.508) (layer "F.Cu") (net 1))
 (segment (start 160.5 94.2078) (end 160.5 90) (width 0.508) (layer "F.Cu") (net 1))
 (segment (start 158.1545 97.836) (end 163.784 97.836) (width 0.254) (layer "F.Cu") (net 35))
 (segment (start 163.784 97.836) (end 165 96.62) (width 0.254) (layer "F.Cu") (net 35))
 (segment (start 163.356612 122.02) (end 158.1545 116.817888) (width 0.254) (layer "F.Cu") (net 24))
 (segment (start 165 122.02) (end 163.356612 122.02) (width 0.254) (layer "F.Cu") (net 24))
 (segment (start 158.1545 116.817888) (end 158.1545 111.806) (width 0.254) (layer "F.Cu") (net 24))
 (segment (start 158.1545 99.106) (end 164.946 99.106) (width 0.254) (layer "F.Cu") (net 34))
 (segment (start 164.946 99.106) (end 165 99.16) (width 0.254) (layer "F.Cu") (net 34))
 (segment (start 158.1545 109.266) (end 159.1578 109.266) (width 0.254) (layer "F.Cu") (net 26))
 (segment (start 159.1578 109.266) (end 160.134 110.2422) (width 0.254) (layer "F.Cu") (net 26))
 (segment (start 161.574 116.94) (end 165 116.94) (width 0.254) (layer "F.Cu") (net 26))
 (segment (start 160.134 115.5) (end 161.574 116.94) (width 0.254) (layer "F.Cu") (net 26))
 (segment (start 160.134 110.2422) (end 160.134 115.5) (width 0.254) (layer "F.Cu") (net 26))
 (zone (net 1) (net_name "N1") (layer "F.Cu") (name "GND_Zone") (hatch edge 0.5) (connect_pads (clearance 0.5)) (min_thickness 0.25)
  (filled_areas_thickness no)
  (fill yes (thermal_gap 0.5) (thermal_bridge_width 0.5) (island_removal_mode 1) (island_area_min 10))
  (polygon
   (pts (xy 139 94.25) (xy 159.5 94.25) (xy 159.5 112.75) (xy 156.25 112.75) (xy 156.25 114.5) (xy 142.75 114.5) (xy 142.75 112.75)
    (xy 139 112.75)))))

